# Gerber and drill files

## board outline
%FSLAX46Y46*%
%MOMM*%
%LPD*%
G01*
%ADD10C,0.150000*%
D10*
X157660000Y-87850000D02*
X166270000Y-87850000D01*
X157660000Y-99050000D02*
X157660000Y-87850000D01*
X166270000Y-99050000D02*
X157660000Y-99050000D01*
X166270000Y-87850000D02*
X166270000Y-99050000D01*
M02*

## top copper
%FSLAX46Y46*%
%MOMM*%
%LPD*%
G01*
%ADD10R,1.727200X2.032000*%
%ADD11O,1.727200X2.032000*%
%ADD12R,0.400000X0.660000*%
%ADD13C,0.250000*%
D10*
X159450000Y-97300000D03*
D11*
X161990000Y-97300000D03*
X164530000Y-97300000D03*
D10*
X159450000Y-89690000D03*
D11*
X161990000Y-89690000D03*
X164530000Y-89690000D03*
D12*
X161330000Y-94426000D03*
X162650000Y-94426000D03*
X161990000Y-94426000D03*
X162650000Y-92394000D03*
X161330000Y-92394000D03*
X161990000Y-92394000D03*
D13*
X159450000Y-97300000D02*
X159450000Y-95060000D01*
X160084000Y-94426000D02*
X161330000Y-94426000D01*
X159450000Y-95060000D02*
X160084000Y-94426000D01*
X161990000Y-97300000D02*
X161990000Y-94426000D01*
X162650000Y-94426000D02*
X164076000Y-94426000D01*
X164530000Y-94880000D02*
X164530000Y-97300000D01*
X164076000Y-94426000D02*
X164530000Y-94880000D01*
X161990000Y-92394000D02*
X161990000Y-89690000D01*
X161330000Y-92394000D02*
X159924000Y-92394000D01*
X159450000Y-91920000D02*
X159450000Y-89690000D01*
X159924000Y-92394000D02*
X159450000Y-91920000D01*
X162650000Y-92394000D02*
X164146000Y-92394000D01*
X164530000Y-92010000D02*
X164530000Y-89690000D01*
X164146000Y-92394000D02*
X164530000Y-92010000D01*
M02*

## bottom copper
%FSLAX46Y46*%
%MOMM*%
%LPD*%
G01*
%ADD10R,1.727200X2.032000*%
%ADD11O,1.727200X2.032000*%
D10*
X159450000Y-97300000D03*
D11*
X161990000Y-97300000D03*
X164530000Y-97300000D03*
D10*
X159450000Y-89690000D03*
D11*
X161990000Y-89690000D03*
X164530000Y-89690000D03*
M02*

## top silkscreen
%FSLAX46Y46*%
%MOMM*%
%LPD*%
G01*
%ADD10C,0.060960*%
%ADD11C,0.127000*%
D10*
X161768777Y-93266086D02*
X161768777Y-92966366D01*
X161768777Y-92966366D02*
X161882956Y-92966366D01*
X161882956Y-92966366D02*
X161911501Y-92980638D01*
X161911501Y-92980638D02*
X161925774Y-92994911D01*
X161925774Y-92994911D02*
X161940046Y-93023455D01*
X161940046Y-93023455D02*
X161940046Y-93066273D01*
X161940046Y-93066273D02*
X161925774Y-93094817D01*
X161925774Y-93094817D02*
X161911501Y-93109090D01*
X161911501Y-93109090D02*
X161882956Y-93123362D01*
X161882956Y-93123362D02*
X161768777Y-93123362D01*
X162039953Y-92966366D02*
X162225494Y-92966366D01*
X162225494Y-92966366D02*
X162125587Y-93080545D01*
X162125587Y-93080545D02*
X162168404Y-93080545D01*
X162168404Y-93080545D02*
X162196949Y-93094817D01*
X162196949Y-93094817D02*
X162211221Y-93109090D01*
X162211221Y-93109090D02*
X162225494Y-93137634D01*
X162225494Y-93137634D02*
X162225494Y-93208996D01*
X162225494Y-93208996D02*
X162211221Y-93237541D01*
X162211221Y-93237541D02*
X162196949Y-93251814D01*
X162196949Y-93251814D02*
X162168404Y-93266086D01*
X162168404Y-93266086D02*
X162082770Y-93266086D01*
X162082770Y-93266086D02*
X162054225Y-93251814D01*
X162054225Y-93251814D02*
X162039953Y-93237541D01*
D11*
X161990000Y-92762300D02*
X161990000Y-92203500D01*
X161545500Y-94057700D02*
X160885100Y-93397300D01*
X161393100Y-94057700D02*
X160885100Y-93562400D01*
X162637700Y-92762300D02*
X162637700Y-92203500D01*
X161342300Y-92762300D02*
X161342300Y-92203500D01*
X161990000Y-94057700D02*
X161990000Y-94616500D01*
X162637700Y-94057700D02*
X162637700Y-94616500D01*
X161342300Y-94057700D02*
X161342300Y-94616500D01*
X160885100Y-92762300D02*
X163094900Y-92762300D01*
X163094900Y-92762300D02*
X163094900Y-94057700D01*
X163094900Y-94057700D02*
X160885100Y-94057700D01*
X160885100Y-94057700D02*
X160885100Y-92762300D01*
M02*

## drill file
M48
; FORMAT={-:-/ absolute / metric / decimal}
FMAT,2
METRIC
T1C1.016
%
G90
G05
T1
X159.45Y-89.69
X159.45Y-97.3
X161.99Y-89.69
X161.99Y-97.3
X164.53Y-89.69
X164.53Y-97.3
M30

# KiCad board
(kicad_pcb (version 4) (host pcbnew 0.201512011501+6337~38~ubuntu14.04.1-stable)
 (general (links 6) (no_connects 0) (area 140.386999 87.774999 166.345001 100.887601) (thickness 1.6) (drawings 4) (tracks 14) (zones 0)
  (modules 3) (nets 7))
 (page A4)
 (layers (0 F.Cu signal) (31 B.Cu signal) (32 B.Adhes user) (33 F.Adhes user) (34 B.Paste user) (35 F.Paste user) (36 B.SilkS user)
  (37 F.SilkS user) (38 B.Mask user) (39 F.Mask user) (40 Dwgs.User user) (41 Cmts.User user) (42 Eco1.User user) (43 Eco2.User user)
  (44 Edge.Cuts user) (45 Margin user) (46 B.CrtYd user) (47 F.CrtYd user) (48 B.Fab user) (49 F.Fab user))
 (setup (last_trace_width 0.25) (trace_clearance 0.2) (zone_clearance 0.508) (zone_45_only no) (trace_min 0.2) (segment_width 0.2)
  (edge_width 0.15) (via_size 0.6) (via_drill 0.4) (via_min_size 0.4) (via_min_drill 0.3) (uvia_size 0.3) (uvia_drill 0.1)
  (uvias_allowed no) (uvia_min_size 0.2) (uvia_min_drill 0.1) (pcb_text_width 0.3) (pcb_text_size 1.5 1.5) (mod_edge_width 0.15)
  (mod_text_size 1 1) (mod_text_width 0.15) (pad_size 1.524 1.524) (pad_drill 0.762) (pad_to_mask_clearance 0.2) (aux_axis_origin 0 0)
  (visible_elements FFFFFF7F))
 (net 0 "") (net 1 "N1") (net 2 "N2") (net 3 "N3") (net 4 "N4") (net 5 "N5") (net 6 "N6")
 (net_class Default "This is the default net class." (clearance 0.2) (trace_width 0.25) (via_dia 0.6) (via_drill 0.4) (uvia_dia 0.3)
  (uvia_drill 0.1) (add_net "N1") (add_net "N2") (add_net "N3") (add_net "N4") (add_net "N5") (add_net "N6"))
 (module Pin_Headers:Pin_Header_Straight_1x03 (layer B.Cu) (at 159.45 97.3 270)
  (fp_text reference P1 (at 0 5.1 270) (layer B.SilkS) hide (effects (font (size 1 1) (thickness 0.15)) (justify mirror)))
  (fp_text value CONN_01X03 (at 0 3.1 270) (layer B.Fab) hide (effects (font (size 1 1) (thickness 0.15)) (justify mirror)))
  (pad 1 thru_hole rect (at 0 0 270) (size 2.032 1.7272) (drill 1.016) (layers *.Cu *.Mask B.SilkS) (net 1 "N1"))
  (pad 2 thru_hole oval (at 0 -2.54 270) (size 2.032 1.7272) (drill 1.016) (layers *.Cu *.Mask B.SilkS) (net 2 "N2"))
  (pad 3 thru_hole oval (at 0 -5.08 270) (size 2.032 1.7272) (drill 1.016) (layers *.Cu *.Mask B.SilkS) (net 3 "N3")))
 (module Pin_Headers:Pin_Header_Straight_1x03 (layer B.Cu) (at 159.45 89.69 270)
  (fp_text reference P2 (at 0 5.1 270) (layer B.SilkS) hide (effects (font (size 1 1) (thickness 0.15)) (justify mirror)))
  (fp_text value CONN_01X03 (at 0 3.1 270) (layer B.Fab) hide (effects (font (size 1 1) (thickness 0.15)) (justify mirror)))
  (pad 1 thru_hole rect (at 0 0 270) (size 2.032 1.7272) (drill 1.016) (layers *.Cu *.Mask B.SilkS) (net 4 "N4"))
  (pad 2 thru_hole oval (at 0 -2.54 270) (size 2.032 1.7272) (drill 1.016) (layers *.Cu *.Mask B.SilkS) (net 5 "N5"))
  (pad 3 thru_hole oval (at 0 -5.08 270) (size 2.032 1.7272) (drill 1.016) (layers *.Cu *.Mask B.SilkS) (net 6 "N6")))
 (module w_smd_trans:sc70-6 (layer F.Cu) (at 161.99 93.41)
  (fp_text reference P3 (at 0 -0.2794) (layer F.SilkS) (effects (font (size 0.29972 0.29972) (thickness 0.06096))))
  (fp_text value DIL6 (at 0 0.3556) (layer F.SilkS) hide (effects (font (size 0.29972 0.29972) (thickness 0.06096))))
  (fp_line (start 0 -0.6477) (end 0 -1.2065) (layer F.SilkS) (width 0.127))
  (fp_line (start -0.4445 0.6477) (end -1.1049 -0.0127) (layer F.SilkS) (width 0.127))
  (fp_line (start -0.5969 0.6477) (end -1.1049 0.1524) (layer F.SilkS) (width 0.127))
  (fp_line (start 0.6477 -0.6477) (end 0.6477 -1.2065) (layer F.SilkS) (width 0.127))
  (fp_line (start -0.6477 -0.6477) (end -0.6477 -1.2065) (layer F.SilkS) (width 0.127))
  (fp_line (start 0 0.6477) (end 0 1.2065) (layer F.SilkS) (width 0.127))
  (fp_line (start 0.6477 0.6477) (end 0.6477 1.2065) (layer F.SilkS) (width 0.127))
  (fp_line (start -0.6477 0.6477) (end -0.6477 1.2065) (layer F.SilkS) (width 0.127))
  (fp_line (start -1.1049 -0.6477) (end 1.1049 -0.6477) (layer F.SilkS) (width 0.127))
  (fp_line (start 1.1049 -0.6477) (end 1.1049 0.6477) (layer F.SilkS) (width 0.127))
  (fp_line (start 1.1049 0.6477) (end -1.1049 0.6477) (layer F.SilkS) (width 0.127))
  (fp_line (start -1.1049 0.6477) (end -1.1049 -0.6477) (layer F.SilkS) (width 0.127))
  (pad 1 smd rect (at -0.66 1.016) (size 0.4 0.66) (layers F.Cu F.Paste F.Mask) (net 1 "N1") (clearance 0.2))
  (pad 3 smd rect (at 0.66 1.016) (size 0.4 0.66) (layers F.Cu F.Paste F.Mask) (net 3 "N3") (clearance 0.2))
  (pad 2 smd rect (at 0 1.016) (size 0.4 0.66) (layers F.Cu F.Paste F.Mask) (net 2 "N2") (clearance 0.2))
  (pad 4 smd rect (at 0.66 -1.016) (size 0.4 0.66) (layers F.Cu F.Paste F.Mask) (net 6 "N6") (clearance 0.2))
  (pad 6 smd rect (at -0.66 -1.016) (size 0.4 0.66) (layers F.Cu F.Paste F.Mask) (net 4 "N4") (clearance 0.2))
  (pad 5 smd rect (at 0 -1.016) (size 0.4 0.66) (layers F.Cu F.Paste F.Mask) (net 5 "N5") (clearance 0.2)))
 (gr_line (start 157.66 87.85) (end 166.27 87.85) (angle 90) (layer Edge.Cuts) (width 0.15))
 (gr_line (start 157.66 99.05) (end 157.66 87.85) (angle 90) (layer Edge.Cuts) (width 0.15))
 (gr_line (start 166.27 99.05) (end 157.66 99.05) (angle 90) (layer Edge.Cuts) (width 0.15))
 (gr_line (start 166.27 87.85) (end 166.27 99.05) (angle 90) (layer Edge.Cuts) (width 0.15))
 (segment (start 159.45 97.3) (end 159.45 95.06) (width 0.25) (layer F.Cu) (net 1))
 (segment (start 160.084 94.426) (end 161.33 94.426) (width 0.25) (layer F.Cu) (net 1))
 (segment (start 159.45 95.06) (end 160.084 94.426) (width 0.25) (layer F.Cu) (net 1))
 (segment (start 161.99 97.3) (end 161.99 94.426) (width 0.25) (layer F.Cu) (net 2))
 (segment (start 162.65 94.426) (end 164.076 94.426) (width 0.25) (layer F.Cu) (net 3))
 (segment (start 164.53 94.88) (end 164.53 97.3) (width 0.25) (layer F.Cu) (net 3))
 (segment (start 164.076 94.426) (end 164.53 94.88) (width 0.25) (layer F.Cu) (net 3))
 (segment (start 161.99 92.394) (end 161.99 89.69) (width 0.25) (layer F.Cu) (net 5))
 (segment (start 161.33 92.394) (end 159.924 92.394) (width 0.25) (layer F.Cu) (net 4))
 (segment (start 159.45 91.92) (end 159.45 89.69) (width 0.25) (layer F.Cu) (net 4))
 (segment (start 159.924 92.394) (end 159.45 91.92) (width 0.25) (layer F.Cu) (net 4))
 (segment (start 162.65 92.394) (end 164.146 92.394) (width 0.25) (layer F.Cu) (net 6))
 (segment (start 164.53 92.01) (end 164.53 89.69) (width 0.25) (layer F.Cu) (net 6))
 (segment (start 164.146 92.394) (end 164.53 92.01) (width 0.25) (layer F.Cu) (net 6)))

